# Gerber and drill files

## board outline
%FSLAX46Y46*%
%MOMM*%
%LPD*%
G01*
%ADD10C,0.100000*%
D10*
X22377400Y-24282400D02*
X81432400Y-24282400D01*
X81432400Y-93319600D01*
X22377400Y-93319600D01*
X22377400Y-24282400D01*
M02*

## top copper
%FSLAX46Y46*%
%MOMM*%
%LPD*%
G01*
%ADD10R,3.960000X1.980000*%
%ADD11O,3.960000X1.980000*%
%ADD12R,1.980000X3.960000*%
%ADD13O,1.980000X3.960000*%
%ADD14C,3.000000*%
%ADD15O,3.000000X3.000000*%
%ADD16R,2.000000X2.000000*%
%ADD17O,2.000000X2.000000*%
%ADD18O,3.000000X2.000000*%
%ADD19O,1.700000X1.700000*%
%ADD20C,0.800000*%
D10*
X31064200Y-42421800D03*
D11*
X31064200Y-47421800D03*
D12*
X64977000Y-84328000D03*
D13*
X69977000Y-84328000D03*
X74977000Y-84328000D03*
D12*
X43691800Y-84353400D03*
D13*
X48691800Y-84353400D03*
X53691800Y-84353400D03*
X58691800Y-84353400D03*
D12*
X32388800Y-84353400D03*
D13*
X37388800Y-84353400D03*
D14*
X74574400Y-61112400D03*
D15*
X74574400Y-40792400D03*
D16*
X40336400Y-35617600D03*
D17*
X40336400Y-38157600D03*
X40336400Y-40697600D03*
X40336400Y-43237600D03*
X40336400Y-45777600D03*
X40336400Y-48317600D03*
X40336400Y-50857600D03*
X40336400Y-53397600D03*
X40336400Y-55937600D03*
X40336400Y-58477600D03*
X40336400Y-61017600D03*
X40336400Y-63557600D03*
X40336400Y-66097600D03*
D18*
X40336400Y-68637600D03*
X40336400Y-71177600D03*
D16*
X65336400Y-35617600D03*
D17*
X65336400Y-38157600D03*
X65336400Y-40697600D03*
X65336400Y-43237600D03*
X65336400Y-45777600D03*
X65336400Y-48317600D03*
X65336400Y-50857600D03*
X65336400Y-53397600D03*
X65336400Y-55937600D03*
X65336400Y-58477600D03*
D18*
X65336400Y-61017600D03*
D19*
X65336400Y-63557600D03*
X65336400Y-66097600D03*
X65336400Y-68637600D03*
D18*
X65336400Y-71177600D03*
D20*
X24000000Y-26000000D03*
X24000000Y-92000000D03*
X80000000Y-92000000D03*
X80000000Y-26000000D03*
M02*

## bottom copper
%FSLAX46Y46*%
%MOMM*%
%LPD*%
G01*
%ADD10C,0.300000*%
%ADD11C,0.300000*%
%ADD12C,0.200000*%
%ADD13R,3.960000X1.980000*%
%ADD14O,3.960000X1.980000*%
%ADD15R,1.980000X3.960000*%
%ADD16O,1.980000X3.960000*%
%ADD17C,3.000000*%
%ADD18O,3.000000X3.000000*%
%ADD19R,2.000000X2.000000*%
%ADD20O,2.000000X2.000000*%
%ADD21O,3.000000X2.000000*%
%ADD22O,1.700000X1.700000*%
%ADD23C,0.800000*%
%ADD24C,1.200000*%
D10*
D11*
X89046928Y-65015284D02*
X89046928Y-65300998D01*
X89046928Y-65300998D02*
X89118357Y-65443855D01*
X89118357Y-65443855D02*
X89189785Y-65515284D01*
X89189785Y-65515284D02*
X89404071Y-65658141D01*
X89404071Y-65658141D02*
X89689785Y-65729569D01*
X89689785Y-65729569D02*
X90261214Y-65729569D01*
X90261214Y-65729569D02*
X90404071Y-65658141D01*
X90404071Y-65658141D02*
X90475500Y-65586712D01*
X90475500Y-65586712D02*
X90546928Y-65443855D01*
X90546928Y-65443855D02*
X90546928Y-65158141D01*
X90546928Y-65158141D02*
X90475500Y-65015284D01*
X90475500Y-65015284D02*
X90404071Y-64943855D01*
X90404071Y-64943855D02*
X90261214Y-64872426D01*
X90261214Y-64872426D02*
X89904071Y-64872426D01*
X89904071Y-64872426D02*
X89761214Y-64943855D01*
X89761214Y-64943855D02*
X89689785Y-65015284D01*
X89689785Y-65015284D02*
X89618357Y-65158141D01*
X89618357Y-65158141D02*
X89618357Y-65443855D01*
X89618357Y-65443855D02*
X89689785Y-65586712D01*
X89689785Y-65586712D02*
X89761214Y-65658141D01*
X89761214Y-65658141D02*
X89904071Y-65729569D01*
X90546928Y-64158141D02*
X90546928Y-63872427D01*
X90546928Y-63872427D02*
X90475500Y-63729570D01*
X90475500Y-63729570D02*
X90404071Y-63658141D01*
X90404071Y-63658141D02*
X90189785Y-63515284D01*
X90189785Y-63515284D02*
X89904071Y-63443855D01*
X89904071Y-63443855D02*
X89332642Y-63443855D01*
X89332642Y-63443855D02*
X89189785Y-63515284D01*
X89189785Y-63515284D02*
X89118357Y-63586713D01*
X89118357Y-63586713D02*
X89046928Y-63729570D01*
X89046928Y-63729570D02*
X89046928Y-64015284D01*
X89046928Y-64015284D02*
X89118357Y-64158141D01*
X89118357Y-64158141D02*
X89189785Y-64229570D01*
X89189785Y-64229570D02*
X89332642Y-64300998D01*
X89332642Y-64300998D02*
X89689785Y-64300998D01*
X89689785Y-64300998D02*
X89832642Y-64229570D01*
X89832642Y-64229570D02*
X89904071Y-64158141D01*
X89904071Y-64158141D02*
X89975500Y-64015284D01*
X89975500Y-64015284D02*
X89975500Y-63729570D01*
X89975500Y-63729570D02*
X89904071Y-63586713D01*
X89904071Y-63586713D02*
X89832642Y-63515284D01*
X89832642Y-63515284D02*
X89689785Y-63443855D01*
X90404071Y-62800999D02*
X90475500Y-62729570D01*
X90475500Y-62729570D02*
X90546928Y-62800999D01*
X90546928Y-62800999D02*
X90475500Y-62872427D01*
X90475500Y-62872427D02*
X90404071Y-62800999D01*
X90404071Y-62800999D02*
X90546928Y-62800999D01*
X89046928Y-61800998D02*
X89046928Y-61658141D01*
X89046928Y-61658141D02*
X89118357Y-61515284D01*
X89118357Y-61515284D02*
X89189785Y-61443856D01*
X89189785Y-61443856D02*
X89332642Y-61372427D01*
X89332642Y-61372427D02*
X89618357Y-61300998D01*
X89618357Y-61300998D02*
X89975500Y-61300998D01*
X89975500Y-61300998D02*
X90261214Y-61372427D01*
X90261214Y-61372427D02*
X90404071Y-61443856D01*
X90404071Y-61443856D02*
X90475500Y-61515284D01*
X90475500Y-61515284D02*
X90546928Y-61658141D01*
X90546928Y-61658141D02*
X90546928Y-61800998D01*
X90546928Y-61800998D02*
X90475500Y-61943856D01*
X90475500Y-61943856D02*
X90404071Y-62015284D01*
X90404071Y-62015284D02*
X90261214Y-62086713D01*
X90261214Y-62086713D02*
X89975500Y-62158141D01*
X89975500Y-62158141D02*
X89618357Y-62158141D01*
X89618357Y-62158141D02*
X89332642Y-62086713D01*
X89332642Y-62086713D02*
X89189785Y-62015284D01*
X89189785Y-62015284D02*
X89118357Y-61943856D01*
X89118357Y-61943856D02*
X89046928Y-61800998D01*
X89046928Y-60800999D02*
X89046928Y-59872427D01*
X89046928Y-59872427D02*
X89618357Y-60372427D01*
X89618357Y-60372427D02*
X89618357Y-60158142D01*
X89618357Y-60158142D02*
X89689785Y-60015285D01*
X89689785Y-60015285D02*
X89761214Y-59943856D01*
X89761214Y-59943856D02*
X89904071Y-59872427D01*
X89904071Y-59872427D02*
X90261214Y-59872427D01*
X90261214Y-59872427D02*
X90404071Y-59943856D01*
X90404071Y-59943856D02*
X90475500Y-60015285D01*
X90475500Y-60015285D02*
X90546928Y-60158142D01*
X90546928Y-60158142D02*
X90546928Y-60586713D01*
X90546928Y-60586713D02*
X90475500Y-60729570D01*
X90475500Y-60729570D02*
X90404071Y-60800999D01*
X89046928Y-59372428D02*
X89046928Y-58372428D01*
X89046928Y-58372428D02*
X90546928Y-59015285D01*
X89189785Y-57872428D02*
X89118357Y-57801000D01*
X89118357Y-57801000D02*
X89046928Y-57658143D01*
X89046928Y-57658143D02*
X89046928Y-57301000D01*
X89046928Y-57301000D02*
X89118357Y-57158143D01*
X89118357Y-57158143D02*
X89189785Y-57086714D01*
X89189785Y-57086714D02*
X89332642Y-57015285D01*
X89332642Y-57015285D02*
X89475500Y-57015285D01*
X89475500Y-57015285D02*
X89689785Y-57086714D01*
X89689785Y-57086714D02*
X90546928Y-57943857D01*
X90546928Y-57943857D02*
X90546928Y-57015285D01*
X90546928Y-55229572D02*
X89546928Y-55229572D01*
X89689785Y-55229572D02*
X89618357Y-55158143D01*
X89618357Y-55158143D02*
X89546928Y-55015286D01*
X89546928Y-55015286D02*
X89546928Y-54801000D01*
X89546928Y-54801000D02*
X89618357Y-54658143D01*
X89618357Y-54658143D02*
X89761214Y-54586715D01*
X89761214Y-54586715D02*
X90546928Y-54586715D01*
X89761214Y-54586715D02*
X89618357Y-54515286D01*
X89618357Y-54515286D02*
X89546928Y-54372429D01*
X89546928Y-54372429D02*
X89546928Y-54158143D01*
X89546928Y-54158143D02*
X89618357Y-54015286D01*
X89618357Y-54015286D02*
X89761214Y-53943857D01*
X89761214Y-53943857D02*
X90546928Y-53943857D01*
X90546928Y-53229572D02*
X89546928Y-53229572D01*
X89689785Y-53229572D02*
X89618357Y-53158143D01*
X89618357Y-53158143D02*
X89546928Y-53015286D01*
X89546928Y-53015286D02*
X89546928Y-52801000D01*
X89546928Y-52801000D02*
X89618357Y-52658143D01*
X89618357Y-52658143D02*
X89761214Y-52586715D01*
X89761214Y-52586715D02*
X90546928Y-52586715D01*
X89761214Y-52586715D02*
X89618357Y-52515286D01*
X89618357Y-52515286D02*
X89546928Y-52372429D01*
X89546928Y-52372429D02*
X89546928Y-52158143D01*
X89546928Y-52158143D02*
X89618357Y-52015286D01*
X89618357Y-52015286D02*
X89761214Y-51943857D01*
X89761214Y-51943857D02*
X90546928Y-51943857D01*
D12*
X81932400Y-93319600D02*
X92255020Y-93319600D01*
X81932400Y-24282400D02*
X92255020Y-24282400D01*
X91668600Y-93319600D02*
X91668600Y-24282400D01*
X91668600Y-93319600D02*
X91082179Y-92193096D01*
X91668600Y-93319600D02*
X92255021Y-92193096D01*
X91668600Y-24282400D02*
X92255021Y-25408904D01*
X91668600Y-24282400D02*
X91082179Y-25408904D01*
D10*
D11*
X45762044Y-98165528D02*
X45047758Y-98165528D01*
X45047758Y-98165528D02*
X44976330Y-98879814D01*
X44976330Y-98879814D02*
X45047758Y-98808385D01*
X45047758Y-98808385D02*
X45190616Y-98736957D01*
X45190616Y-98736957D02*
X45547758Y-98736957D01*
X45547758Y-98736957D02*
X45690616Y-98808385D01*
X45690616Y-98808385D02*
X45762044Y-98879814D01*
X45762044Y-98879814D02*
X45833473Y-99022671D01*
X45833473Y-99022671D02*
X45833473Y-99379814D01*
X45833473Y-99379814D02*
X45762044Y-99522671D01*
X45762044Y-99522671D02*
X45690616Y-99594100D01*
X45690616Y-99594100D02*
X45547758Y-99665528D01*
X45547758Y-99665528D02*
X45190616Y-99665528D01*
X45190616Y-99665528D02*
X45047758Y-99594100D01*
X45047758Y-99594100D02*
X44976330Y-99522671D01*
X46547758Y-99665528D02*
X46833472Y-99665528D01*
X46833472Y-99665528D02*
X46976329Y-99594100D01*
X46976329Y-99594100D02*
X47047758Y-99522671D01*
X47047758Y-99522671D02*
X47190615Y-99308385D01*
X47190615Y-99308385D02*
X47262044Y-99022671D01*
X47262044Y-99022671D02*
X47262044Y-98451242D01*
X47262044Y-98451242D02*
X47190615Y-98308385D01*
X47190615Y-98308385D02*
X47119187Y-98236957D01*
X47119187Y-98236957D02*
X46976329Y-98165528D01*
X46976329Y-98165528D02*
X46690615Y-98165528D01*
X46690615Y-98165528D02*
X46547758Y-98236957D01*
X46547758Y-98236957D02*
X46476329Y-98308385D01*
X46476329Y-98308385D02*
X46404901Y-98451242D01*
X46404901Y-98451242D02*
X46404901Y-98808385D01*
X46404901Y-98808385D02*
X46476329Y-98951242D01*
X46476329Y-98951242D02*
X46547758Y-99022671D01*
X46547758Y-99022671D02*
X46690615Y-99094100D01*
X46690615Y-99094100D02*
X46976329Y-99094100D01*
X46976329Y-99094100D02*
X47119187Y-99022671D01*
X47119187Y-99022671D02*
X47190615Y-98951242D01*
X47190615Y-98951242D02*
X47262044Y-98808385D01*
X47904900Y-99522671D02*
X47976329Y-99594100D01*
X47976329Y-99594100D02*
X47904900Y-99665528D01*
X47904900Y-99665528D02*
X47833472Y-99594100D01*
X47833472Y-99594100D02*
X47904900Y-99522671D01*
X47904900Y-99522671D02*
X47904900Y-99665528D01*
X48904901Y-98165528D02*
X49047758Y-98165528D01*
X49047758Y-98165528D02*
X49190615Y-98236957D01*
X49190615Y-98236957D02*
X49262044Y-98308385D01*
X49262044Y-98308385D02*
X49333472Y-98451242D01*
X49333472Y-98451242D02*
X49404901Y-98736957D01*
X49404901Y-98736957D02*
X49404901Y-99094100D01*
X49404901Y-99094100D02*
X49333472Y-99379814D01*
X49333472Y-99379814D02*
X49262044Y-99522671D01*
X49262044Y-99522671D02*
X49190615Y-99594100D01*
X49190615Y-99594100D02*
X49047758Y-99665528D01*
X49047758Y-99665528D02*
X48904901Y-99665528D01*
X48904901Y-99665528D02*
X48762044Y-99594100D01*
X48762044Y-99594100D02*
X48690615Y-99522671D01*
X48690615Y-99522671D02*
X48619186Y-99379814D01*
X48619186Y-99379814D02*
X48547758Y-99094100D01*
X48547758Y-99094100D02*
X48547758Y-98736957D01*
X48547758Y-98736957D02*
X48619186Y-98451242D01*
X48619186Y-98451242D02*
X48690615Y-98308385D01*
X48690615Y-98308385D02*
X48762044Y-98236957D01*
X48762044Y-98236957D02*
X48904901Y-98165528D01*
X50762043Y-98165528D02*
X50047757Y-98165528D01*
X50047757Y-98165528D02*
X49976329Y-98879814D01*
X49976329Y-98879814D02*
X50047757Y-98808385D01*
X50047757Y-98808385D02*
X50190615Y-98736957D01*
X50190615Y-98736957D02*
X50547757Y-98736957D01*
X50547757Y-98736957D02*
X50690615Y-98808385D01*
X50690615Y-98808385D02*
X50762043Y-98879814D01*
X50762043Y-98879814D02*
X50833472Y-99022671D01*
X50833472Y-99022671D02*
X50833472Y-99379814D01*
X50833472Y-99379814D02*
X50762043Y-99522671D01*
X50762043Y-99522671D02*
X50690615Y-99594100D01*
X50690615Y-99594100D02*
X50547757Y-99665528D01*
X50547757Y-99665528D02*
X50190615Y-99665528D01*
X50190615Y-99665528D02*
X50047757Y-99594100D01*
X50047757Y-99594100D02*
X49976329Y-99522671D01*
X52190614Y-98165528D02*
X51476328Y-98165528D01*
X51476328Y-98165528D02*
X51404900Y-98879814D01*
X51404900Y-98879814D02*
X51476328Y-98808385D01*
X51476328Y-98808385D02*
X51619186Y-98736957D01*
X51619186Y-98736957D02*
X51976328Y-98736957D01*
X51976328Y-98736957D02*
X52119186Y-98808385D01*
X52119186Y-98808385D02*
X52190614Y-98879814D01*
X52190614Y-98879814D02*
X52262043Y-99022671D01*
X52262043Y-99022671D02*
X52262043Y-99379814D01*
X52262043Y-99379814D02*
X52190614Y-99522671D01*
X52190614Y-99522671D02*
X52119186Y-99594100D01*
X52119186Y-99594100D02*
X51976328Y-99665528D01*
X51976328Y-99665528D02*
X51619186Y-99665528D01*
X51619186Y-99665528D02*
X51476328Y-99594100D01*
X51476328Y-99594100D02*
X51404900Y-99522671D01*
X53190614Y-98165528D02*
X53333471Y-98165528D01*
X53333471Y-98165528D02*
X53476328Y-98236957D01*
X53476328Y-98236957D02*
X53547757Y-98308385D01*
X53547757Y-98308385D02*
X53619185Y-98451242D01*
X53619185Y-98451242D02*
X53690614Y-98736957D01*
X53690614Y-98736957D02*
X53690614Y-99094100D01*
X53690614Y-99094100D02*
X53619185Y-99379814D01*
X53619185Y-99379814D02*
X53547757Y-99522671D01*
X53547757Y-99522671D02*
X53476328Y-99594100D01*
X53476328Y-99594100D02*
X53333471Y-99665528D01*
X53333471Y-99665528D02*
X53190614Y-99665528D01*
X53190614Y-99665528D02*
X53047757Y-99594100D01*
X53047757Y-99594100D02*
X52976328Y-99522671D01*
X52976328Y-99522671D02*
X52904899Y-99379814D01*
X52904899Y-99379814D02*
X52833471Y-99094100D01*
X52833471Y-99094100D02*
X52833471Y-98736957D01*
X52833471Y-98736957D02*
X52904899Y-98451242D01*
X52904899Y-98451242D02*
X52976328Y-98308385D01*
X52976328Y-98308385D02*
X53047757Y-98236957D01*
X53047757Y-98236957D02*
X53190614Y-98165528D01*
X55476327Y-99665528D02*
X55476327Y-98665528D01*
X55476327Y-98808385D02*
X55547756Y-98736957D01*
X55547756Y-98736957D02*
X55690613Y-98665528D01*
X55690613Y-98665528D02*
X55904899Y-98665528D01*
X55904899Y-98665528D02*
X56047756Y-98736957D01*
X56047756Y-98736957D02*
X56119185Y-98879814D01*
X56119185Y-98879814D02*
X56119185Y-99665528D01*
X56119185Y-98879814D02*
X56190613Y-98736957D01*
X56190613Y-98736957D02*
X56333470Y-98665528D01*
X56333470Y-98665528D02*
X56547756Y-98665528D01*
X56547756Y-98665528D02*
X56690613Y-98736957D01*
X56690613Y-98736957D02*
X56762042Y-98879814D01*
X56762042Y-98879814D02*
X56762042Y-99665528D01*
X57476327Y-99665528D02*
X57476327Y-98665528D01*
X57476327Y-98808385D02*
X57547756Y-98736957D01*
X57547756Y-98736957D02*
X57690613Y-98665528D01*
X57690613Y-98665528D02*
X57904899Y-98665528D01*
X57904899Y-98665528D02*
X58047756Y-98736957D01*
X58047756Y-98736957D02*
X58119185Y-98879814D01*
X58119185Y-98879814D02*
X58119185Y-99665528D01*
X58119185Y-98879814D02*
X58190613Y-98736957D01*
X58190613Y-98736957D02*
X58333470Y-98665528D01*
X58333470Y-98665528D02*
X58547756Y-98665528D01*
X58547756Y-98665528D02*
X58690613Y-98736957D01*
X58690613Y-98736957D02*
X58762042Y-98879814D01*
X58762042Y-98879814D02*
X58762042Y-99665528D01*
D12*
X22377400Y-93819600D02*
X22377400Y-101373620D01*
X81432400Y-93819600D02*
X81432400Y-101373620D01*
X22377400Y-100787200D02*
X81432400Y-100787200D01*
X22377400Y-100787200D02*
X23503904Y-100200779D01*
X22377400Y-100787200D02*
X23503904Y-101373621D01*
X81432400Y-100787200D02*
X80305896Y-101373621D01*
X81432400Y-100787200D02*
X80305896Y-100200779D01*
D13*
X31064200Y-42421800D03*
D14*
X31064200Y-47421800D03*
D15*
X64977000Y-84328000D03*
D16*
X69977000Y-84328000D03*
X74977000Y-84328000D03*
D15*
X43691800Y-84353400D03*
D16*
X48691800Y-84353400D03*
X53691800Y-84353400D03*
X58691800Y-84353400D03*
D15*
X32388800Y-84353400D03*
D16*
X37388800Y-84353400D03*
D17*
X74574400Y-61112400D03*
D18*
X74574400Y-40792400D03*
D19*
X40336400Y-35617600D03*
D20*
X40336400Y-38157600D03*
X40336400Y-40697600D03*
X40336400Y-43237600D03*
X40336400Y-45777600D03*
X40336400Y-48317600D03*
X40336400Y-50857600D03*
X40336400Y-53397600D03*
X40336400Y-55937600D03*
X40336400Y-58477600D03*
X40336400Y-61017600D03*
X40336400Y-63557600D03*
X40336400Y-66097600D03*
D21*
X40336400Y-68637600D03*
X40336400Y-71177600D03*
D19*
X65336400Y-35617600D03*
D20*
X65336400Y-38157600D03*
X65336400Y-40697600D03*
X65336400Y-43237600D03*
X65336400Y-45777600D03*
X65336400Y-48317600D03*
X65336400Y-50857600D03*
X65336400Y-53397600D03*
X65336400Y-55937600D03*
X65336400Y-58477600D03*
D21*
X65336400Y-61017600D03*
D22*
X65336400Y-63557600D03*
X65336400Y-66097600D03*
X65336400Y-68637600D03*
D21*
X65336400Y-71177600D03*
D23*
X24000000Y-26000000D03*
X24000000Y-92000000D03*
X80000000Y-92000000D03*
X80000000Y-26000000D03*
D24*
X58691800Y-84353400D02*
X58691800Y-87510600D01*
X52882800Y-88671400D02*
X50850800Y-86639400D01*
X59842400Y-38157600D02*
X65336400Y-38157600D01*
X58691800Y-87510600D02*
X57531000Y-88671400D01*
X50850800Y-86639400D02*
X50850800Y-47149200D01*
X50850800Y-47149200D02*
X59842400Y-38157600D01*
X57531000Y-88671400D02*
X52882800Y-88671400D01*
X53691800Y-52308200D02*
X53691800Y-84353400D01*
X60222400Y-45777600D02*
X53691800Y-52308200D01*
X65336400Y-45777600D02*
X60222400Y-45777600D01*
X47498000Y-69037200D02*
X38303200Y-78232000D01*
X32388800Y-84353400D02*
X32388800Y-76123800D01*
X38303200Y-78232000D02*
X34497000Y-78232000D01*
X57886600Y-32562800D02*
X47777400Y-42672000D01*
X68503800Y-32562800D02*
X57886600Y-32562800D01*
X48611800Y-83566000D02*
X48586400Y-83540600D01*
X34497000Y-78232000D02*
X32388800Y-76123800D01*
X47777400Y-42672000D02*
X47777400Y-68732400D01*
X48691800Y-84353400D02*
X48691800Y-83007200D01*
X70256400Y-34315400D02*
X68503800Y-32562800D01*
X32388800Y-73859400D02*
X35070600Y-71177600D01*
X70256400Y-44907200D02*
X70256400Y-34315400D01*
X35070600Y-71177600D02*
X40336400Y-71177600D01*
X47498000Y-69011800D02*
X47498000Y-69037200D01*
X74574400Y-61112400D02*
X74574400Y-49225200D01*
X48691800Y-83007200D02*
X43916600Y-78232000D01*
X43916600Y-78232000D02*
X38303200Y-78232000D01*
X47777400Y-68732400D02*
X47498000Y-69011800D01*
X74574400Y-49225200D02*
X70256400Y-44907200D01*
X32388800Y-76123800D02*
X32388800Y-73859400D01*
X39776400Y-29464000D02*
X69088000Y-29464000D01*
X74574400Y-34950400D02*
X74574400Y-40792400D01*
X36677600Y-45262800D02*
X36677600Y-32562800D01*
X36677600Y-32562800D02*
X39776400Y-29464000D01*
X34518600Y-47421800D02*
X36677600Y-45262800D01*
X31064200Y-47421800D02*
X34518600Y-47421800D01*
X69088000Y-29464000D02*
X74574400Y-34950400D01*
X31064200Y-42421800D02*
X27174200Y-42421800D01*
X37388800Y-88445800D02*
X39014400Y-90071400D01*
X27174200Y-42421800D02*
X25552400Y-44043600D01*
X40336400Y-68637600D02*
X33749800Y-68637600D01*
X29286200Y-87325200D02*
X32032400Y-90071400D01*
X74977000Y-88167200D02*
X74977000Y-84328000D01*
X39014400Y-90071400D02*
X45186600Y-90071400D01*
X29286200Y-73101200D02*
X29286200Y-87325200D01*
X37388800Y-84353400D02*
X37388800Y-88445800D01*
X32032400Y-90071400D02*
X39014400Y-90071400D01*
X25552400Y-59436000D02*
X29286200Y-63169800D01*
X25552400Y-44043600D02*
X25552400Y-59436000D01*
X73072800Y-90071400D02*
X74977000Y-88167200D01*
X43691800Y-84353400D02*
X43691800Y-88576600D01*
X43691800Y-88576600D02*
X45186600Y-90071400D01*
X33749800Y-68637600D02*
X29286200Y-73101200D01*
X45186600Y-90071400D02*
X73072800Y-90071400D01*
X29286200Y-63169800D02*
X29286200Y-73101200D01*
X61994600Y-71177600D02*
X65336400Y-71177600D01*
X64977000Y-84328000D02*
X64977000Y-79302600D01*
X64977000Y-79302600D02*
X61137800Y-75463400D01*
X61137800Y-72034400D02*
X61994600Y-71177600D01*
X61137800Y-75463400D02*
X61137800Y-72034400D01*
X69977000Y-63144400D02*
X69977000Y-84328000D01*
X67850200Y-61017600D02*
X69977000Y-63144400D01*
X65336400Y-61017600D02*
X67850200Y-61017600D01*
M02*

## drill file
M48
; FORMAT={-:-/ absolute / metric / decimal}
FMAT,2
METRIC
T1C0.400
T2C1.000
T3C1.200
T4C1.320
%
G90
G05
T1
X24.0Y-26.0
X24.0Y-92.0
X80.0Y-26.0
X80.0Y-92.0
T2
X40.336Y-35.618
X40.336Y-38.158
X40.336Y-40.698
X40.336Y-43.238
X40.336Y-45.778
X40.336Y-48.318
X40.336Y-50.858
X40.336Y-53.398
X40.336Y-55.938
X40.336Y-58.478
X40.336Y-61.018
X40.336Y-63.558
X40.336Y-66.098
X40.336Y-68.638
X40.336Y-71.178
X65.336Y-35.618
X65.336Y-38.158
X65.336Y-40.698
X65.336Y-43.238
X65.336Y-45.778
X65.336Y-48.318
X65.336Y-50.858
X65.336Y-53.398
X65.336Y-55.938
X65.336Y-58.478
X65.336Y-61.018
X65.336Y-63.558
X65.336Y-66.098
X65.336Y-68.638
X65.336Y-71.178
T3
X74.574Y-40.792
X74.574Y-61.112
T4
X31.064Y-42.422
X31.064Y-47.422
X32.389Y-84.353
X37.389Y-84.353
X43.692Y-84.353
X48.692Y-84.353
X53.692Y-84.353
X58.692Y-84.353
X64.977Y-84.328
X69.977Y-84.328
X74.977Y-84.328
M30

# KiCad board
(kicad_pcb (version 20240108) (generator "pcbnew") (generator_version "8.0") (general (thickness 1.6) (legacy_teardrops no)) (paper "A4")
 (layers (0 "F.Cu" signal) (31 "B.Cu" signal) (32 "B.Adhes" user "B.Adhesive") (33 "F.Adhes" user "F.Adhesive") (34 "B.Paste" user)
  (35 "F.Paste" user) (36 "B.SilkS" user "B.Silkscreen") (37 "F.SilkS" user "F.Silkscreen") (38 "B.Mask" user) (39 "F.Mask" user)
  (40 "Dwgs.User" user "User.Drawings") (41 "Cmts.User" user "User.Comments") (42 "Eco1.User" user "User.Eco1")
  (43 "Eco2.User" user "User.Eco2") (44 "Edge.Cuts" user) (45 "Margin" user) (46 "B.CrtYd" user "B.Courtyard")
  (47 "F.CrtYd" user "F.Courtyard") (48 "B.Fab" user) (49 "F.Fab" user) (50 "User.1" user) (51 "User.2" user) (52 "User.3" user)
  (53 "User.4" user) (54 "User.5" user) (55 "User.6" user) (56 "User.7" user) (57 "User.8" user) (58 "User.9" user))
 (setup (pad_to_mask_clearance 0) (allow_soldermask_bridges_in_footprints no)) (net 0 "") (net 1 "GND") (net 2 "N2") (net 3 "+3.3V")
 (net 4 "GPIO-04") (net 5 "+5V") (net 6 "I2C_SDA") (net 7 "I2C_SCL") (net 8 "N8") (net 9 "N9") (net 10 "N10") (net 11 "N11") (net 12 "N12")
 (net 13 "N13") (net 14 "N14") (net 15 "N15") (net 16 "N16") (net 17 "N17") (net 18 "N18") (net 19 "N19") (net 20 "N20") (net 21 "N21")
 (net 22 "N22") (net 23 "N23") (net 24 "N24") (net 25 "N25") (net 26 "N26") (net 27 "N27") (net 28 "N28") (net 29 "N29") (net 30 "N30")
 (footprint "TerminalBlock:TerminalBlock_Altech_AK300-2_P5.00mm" (layer "F.Cu") (at 31.0642 42.4218 -90)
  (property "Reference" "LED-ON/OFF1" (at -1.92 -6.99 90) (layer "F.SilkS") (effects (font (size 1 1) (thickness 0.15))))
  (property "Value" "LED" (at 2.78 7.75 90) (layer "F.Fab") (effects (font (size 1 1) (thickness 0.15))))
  (pad "1" thru_hole rect (at 0 0 270) (size 1.98 3.96) (drill 1.32) (layers "*.Cu" "*.Mask") (remove_unused_layers no) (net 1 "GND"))
  (pad "2" thru_hole oval (at 5 0 270) (size 1.98 3.96) (drill 1.32) (layers "*.Cu" "*.Mask") (remove_unused_layers no) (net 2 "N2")))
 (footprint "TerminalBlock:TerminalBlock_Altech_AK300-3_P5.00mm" (layer "F.Cu") (at 64.977 84.328)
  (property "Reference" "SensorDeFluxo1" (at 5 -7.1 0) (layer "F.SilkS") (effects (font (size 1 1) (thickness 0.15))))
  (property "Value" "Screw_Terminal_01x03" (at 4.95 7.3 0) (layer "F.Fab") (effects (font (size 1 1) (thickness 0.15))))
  (pad "1" thru_hole rect (at 0 0) (size 1.98 3.96) (drill 1.32) (layers "*.Cu" "*.Mask") (remove_unused_layers no) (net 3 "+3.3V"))
  (pad "2" thru_hole oval (at 5 0) (size 1.98 3.96) (drill 1.32) (layers "*.Cu" "*.Mask") (remove_unused_layers no) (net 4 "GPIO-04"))
  (pad "3" thru_hole oval (at 10 0) (size 1.98 3.96) (drill 1.32) (layers "*.Cu" "*.Mask") (remove_unused_layers no) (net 1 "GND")))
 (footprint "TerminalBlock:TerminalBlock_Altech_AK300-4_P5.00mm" (layer "F.Cu") (at 43.6918 84.3534)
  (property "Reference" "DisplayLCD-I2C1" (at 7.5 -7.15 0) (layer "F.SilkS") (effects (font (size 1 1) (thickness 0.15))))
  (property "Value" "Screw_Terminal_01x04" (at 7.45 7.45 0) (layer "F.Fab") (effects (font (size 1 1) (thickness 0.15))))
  (pad "1" thru_hole rect (at 0 0) (size 1.98 3.96) (drill 1.32) (layers "*.Cu" "*.Mask") (remove_unused_layers no) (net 1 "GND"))
  (pad "2" thru_hole oval (at 5 0) (size 1.98 3.96) (drill 1.32) (layers "*.Cu" "*.Mask") (remove_unused_layers no) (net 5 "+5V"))
  (pad "3" thru_hole oval (at 10 0) (size 1.98 3.96) (drill 1.32) (layers "*.Cu" "*.Mask") (remove_unused_layers no) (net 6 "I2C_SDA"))
  (pad "4" thru_hole oval (at 15 0) (size 1.98 3.96) (drill 1.32) (layers "*.Cu" "*.Mask") (remove_unused_layers no) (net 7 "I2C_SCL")))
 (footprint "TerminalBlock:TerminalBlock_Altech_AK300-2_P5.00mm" (layer "F.Cu") (at 32.3888 84.3534)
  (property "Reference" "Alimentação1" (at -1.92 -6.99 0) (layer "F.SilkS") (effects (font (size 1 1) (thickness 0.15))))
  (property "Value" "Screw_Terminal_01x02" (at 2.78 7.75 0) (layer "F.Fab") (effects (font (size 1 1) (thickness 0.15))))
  (pad "1" thru_hole rect (at 0 0) (size 1.98 3.96) (drill 1.32) (layers "*.Cu" "*.Mask") (remove_unused_layers no) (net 5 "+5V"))
  (pad "2" thru_hole oval (at 5 0) (size 1.98 3.96) (drill 1.32) (layers "*.Cu" "*.Mask") (remove_unused_layers no) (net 1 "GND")))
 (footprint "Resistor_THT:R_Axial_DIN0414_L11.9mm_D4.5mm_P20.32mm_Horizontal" (layer "F.Cu") (at 74.5744 61.1124 90)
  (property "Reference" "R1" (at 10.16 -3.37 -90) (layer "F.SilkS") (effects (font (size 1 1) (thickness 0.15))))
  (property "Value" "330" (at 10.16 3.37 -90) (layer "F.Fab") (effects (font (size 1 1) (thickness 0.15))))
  (pad "1" thru_hole circle (at 0 0 90) (size 3 3) (drill 1.2) (layers "*.Cu" "*.Mask") (remove_unused_layers no) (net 5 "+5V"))
  (pad "2" thru_hole oval (at 20.32 0 90) (size 3 3) (drill 1.2) (layers "*.Cu" "*.Mask") (remove_unused_layers no) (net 2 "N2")))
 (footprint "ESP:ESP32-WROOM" (layer "F.Cu") (at 51.7114 54.4676)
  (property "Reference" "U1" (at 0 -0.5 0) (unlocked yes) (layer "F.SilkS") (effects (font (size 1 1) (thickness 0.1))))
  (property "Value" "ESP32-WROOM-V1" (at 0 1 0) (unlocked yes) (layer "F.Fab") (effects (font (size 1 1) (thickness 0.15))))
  (pad "1" thru_hole rect (at -11.375 -18.85) (size 2 2) (drill 1) (layers "*.Cu" "*.Mask") (remove_unused_layers no) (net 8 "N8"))
  (pad "2" thru_hole oval (at -11.375 -16.31) (size 2 2) (drill 1) (layers "*.Cu" "*.Mask") (remove_unused_layers no) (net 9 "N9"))
  (pad "3" thru_hole oval (at -11.375 -13.77) (size 2 2) (drill 1) (layers "*.Cu" "*.Mask") (remove_unused_layers no) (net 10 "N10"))
  (pad "4" thru_hole oval (at -11.375 -11.23) (size 2 2) (drill 1) (layers "*.Cu" "*.Mask") (remove_unused_layers no) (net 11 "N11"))
  (pad "5" thru_hole oval (at -11.375 -8.69) (size 2 2) (drill 1) (layers "*.Cu" "*.Mask") (remove_unused_layers no) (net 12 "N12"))
  (pad "6" thru_hole oval (at -11.375 -6.15) (size 2 2) (drill 1) (layers "*.Cu" "*.Mask") (remove_unused_layers no) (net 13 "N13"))
  (pad "7" thru_hole oval (at -11.375 -3.61) (size 2 2) (drill 1) (layers "*.Cu" "*.Mask") (remove_unused_layers no) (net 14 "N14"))
  (pad "8" thru_hole oval (at -11.375 -1.07) (size 2 2) (drill 1) (layers "*.Cu" "*.Mask") (remove_unused_layers no) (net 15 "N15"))
  (pad "9" thru_hole oval (at -11.375 1.47) (size 2 2) (drill 1) (layers "*.Cu" "*.Mask") (remove_unused_layers no) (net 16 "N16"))
  (pad "10" thru_hole oval (at -11.375 4.01) (size 2 2) (drill 1) (layers "*.Cu" "*.Mask") (remove_unused_layers no) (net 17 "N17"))
  (pad "11" thru_hole oval (at -11.375 6.55) (size 2 2) (drill 1) (layers "*.Cu" "*.Mask") (remove_unused_layers no) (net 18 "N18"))
  (pad "12" thru_hole oval (at -11.375 9.09) (size 2 2) (drill 1) (layers "*.Cu" "*.Mask") (remove_unused_layers no) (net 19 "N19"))
  (pad "13" thru_hole oval (at -11.375 11.63) (size 2 2) (drill 1) (layers "*.Cu" "*.Mask") (remove_unused_layers no) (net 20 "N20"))
  (pad "14" thru_hole oval (at -11.375 14.17) (size 3 2) (drill 1) (layers "*.Cu" "*.Mask") (remove_unused_layers no) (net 1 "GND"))
  (pad "15" thru_hole oval (at -11.375 16.71) (size 3 2) (drill 1) (layers "*.Cu" "*.Mask") (remove_unused_layers no) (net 5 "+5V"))
  (pad "16" thru_hole rect (at 13.625 -18.85) (size 2 2) (drill 1) (layers "*.Cu" "*.Mask") (remove_unused_layers no) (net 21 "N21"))
  (pad "17" thru_hole oval (at 13.625 -16.31) (size 2 2) (drill 1) (layers "*.Cu" "*.Mask") (remove_unused_layers no) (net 7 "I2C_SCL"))
  (pad "18" thru_hole oval (at 13.625 -13.77) (size 2 2) (drill 1) (layers "*.Cu" "*.Mask") (remove_unused_layers no) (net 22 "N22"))
  (pad "19" thru_hole oval (at 13.625 -11.23) (size 2 2) (drill 1) (layers "*.Cu" "*.Mask") (remove_unused_layers no) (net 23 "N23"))
  (pad "20" thru_hole oval (at 13.625 -8.69) (size 2 2) (drill 1) (layers "*.Cu" "*.Mask") (remove_unused_layers no) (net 6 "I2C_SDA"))
  (pad "21" thru_hole oval (at 13.625 -6.15) (size 2 2) (drill 1) (layers "*.Cu" "*.Mask") (remove_unused_layers no) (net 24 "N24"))
  (pad "22" thru_hole oval (at 13.625 -3.61) (size 2 2) (drill 1) (layers "*.Cu" "*.Mask") (remove_unused_layers no) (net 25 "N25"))
  (pad "23" thru_hole oval (at 13.625 -1.07) (size 2 2) (drill 1) (layers "*.Cu" "*.Mask") (remove_unused_layers no) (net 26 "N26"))
  (pad "24" thru_hole oval (at 13.625 1.47) (size 2 2) (drill 1) (layers "*.Cu" "*.Mask") (remove_unused_layers no) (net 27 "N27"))
  (pad "25" thru_hole oval (at 13.625 4.01) (size 2 2) (drill 1) (layers "*.Cu" "*.Mask") (remove_unused_layers no) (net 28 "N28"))
  (pad "26" thru_hole oval (at 13.625 6.55) (size 3 2) (drill 1) (layers "*.Cu" "*.Mask") (remove_unused_layers no) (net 4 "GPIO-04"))
  (pad "27" thru_hole oval (at 13.625 9.09) (size 1.7 1.7) (drill 1) (layers "*.Cu" "*.Mask") (remove_unused_layers no) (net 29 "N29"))
  (pad "28" thru_hole oval (at 13.625 11.63) (size 1.7 1.7) (drill 1) (layers "*.Cu" "*.Mask") (remove_unused_layers no) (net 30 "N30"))
  (pad "29" thru_hole oval (at 13.625 14.17) (size 1.7 1.7) (drill 1) (layers "*.Cu" "*.Mask") (remove_unused_layers no) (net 1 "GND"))
  (pad "30" thru_hole oval (at 13.625 16.71) (size 3 2) (drill 1) (layers "*.Cu" "*.Mask") (remove_unused_layers no) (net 3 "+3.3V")))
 (gr_rect (start 22.3774 24.2824) (end 81.4324 93.3196) (stroke (width 0.1) (type default)) (fill none) (layer "Edge.Cuts"))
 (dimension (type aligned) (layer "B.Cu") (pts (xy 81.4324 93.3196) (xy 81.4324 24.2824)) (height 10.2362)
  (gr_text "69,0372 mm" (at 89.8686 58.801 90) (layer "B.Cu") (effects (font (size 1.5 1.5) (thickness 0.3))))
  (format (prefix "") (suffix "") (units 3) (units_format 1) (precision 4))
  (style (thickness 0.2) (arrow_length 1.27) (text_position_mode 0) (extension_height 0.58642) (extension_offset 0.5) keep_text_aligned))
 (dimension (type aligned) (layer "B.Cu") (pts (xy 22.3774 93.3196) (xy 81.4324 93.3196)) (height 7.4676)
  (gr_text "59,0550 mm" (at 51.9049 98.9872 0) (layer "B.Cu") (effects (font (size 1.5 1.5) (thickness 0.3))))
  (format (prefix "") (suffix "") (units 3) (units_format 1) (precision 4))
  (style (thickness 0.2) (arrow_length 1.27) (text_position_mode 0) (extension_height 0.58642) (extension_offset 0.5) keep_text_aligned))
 (via (at 24 26) (size 0.8) (drill 0.4) (layers "F.Cu" "B.Cu") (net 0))
 (via (at 24 92) (size 0.8) (drill 0.4) (layers "F.Cu" "B.Cu") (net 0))
 (via (at 80 92) (size 0.8) (drill 0.4) (layers "F.Cu" "B.Cu") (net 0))
 (via (at 80 26) (size 0.8) (drill 0.4) (layers "F.Cu" "B.Cu") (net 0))
 (segment (start 58.6918 84.3534) (end 58.6918 87.5106) (width 1.2) (layer "B.Cu") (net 7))
 (segment (start 52.8828 88.6714) (end 50.8508 86.6394) (width 1.2) (layer "B.Cu") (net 7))
 (segment (start 59.8424 38.1576) (end 65.3364 38.1576) (width 1.2) (layer "B.Cu") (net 7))
 (segment (start 58.6918 87.5106) (end 57.531 88.6714) (width 1.2) (layer "B.Cu") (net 7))
 (segment (start 50.8508 86.6394) (end 50.8508 47.1492) (width 1.2) (layer "B.Cu") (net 7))
 (segment (start 50.8508 47.1492) (end 59.8424 38.1576) (width 1.2) (layer "B.Cu") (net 7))
 (segment (start 57.531 88.6714) (end 52.8828 88.6714) (width 1.2) (layer "B.Cu") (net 7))
 (segment (start 53.6918 52.3082) (end 53.6918 84.3534) (width 1.2) (layer "B.Cu") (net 6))
 (segment (start 60.2224 45.7776) (end 53.6918 52.3082) (width 1.2) (layer "B.Cu") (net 6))
 (segment (start 65.3364 45.7776) (end 60.2224 45.7776) (width 1.2) (layer "B.Cu") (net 6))
 (segment (start 47.498 69.0372) (end 38.3032 78.232) (width 1.2) (layer "B.Cu") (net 5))
 (segment (start 32.3888 84.3534) (end 32.3888 76.1238) (width 1.2) (layer "B.Cu") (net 5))
 (segment (start 38.3032 78.232) (end 34.497 78.232) (width 1.2) (layer "B.Cu") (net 5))
 (segment (start 57.8866 32.5628) (end 47.7774 42.672) (width 1.2) (layer "B.Cu") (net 5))
 (segment (start 68.5038 32.5628) (end 57.8866 32.5628) (width 1.2) (layer "B.Cu") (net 5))
 (segment (start 48.6118 83.566) (end 48.5864 83.5406) (width 1.2) (layer "B.Cu") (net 5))
 (segment (start 34.497 78.232) (end 32.3888 76.1238) (width 1.2) (layer "B.Cu") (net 5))
 (segment (start 47.7774 42.672) (end 47.7774 68.7324) (width 1.2) (layer "B.Cu") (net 5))
 (segment (start 48.6918 84.3534) (end 48.6918 83.0072) (width 1.2) (layer "B.Cu") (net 5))
 (segment (start 70.2564 34.3154) (end 68.5038 32.5628) (width 1.2) (layer "B.Cu") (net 5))
 (segment (start 32.3888 73.8594) (end 35.0706 71.1776) (width 1.2) (layer "B.Cu") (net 5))
 (segment (start 70.2564 44.9072) (end 70.2564 34.3154) (width 1.2) (layer "B.Cu") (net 5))
 (segment (start 35.0706 71.1776) (end 40.3364 71.1776) (width 1.2) (layer "B.Cu") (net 5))
 (segment (start 47.498 69.0118) (end 47.498 69.0372) (width 1.2) (layer "B.Cu") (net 5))
 (segment (start 74.5744 61.1124) (end 74.5744 49.2252) (width 1.2) (layer "B.Cu") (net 5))
 (segment (start 48.6918 83.0072) (end 43.9166 78.232) (width 1.2) (layer "B.Cu") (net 5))
 (segment (start 43.9166 78.232) (end 38.3032 78.232) (width 1.2) (layer "B.Cu") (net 5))
 (segment (start 47.7774 68.7324) (end 47.498 69.0118) (width 1.2) (layer "B.Cu") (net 5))
 (segment (start 74.5744 49.2252) (end 70.2564 44.9072) (width 1.2) (layer "B.Cu") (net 5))
 (segment (start 32.3888 76.1238) (end 32.3888 73.8594) (width 1.2) (layer "B.Cu") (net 5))
 (segment (start 39.7764 29.464) (end 69.088 29.464) (width 1.2) (layer "B.Cu") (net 2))
 (segment (start 74.5744 34.9504) (end 74.5744 40.7924) (width 1.2) (layer "B.Cu") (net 2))
 (segment (start 36.6776 45.2628) (end 36.6776 32.5628) (width 1.2) (layer "B.Cu") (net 2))
 (segment (start 36.6776 32.5628) (end 39.7764 29.464) (width 1.2) (layer "B.Cu") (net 2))
 (segment (start 34.5186 47.4218) (end 36.6776 45.2628) (width 1.2) (layer "B.Cu") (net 2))
 (segment (start 31.0642 47.4218) (end 34.5186 47.4218) (width 1.2) (layer "B.Cu") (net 2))
 (segment (start 69.088 29.464) (end 74.5744 34.9504) (width 1.2) (layer "B.Cu") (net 2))
 (segment (start 31.0642 42.4218) (end 27.1742 42.4218) (width 1.2) (layer "B.Cu") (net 1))
 (segment (start 37.3888 88.4458) (end 39.0144 90.0714) (width 1.2) (layer "B.Cu") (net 1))
 (segment (start 27.1742 42.4218) (end 25.5524 44.0436) (width 1.2) (layer "B.Cu") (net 1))
 (segment (start 40.3364 68.6376) (end 33.7498 68.6376) (width 1.2) (layer "B.Cu") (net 1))
 (segment (start 29.2862 87.3252) (end 32.0324 90.0714) (width 1.2) (layer "B.Cu") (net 1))
 (segment (start 74.977 88.1672) (end 74.977 84.328) (width 1.2) (layer "B.Cu") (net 1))
 (segment (start 39.0144 90.0714) (end 45.1866 90.0714) (width 1.2) (layer "B.Cu") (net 1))
 (segment (start 29.2862 73.1012) (end 29.2862 87.3252) (width 1.2) (layer "B.Cu") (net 1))
 (segment (start 37.3888 84.3534) (end 37.3888 88.4458) (width 1.2) (layer "B.Cu") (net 1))
 (segment (start 32.0324 90.0714) (end 39.0144 90.0714) (width 1.2) (layer "B.Cu") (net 1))
 (segment (start 25.5524 59.436) (end 29.2862 63.1698) (width 1.2) (layer "B.Cu") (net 1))
 (segment (start 25.5524 44.0436) (end 25.5524 59.436) (width 1.2) (layer "B.Cu") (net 1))
 (segment (start 73.0728 90.0714) (end 74.977 88.1672) (width 1.2) (layer "B.Cu") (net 1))
 (segment (start 43.6918 84.3534) (end 43.6918 88.5766) (width 1.2) (layer "B.Cu") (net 1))
 (segment (start 43.6918 88.5766) (end 45.1866 90.0714) (width 1.2) (layer "B.Cu") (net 1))
 (segment (start 33.7498 68.6376) (end 29.2862 73.1012) (width 1.2) (layer "B.Cu") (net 1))
 (segment (start 45.1866 90.0714) (end 73.0728 90.0714) (width 1.2) (layer "B.Cu") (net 1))
 (segment (start 29.2862 63.1698) (end 29.2862 73.1012) (width 1.2) (layer "B.Cu") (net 1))
 (segment (start 61.9946 71.1776) (end 65.3364 71.1776) (width 1.2) (layer "B.Cu") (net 3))
 (segment (start 64.977 84.328) (end 64.977 79.3026) (width 1.2) (layer "B.Cu") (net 3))
 (segment (start 64.977 79.3026) (end 61.1378 75.4634) (width 1.2) (layer "B.Cu") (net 3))
 (segment (start 61.1378 72.0344) (end 61.9946 71.1776) (width 1.2) (layer "B.Cu") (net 3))
 (segment (start 61.1378 75.4634) (end 61.1378 72.0344) (width 1.2) (layer "B.Cu") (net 3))
 (segment (start 69.977 63.1444) (end 69.977 84.328) (width 1.2) (layer "B.Cu") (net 4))
 (segment (start 67.8502 61.0176) (end 69.977 63.1444) (width 1.2) (layer "B.Cu") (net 4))
 (segment (start 65.3364 61.0176) (end 67.8502 61.0176) (width 1.2) (layer "B.Cu") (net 4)))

